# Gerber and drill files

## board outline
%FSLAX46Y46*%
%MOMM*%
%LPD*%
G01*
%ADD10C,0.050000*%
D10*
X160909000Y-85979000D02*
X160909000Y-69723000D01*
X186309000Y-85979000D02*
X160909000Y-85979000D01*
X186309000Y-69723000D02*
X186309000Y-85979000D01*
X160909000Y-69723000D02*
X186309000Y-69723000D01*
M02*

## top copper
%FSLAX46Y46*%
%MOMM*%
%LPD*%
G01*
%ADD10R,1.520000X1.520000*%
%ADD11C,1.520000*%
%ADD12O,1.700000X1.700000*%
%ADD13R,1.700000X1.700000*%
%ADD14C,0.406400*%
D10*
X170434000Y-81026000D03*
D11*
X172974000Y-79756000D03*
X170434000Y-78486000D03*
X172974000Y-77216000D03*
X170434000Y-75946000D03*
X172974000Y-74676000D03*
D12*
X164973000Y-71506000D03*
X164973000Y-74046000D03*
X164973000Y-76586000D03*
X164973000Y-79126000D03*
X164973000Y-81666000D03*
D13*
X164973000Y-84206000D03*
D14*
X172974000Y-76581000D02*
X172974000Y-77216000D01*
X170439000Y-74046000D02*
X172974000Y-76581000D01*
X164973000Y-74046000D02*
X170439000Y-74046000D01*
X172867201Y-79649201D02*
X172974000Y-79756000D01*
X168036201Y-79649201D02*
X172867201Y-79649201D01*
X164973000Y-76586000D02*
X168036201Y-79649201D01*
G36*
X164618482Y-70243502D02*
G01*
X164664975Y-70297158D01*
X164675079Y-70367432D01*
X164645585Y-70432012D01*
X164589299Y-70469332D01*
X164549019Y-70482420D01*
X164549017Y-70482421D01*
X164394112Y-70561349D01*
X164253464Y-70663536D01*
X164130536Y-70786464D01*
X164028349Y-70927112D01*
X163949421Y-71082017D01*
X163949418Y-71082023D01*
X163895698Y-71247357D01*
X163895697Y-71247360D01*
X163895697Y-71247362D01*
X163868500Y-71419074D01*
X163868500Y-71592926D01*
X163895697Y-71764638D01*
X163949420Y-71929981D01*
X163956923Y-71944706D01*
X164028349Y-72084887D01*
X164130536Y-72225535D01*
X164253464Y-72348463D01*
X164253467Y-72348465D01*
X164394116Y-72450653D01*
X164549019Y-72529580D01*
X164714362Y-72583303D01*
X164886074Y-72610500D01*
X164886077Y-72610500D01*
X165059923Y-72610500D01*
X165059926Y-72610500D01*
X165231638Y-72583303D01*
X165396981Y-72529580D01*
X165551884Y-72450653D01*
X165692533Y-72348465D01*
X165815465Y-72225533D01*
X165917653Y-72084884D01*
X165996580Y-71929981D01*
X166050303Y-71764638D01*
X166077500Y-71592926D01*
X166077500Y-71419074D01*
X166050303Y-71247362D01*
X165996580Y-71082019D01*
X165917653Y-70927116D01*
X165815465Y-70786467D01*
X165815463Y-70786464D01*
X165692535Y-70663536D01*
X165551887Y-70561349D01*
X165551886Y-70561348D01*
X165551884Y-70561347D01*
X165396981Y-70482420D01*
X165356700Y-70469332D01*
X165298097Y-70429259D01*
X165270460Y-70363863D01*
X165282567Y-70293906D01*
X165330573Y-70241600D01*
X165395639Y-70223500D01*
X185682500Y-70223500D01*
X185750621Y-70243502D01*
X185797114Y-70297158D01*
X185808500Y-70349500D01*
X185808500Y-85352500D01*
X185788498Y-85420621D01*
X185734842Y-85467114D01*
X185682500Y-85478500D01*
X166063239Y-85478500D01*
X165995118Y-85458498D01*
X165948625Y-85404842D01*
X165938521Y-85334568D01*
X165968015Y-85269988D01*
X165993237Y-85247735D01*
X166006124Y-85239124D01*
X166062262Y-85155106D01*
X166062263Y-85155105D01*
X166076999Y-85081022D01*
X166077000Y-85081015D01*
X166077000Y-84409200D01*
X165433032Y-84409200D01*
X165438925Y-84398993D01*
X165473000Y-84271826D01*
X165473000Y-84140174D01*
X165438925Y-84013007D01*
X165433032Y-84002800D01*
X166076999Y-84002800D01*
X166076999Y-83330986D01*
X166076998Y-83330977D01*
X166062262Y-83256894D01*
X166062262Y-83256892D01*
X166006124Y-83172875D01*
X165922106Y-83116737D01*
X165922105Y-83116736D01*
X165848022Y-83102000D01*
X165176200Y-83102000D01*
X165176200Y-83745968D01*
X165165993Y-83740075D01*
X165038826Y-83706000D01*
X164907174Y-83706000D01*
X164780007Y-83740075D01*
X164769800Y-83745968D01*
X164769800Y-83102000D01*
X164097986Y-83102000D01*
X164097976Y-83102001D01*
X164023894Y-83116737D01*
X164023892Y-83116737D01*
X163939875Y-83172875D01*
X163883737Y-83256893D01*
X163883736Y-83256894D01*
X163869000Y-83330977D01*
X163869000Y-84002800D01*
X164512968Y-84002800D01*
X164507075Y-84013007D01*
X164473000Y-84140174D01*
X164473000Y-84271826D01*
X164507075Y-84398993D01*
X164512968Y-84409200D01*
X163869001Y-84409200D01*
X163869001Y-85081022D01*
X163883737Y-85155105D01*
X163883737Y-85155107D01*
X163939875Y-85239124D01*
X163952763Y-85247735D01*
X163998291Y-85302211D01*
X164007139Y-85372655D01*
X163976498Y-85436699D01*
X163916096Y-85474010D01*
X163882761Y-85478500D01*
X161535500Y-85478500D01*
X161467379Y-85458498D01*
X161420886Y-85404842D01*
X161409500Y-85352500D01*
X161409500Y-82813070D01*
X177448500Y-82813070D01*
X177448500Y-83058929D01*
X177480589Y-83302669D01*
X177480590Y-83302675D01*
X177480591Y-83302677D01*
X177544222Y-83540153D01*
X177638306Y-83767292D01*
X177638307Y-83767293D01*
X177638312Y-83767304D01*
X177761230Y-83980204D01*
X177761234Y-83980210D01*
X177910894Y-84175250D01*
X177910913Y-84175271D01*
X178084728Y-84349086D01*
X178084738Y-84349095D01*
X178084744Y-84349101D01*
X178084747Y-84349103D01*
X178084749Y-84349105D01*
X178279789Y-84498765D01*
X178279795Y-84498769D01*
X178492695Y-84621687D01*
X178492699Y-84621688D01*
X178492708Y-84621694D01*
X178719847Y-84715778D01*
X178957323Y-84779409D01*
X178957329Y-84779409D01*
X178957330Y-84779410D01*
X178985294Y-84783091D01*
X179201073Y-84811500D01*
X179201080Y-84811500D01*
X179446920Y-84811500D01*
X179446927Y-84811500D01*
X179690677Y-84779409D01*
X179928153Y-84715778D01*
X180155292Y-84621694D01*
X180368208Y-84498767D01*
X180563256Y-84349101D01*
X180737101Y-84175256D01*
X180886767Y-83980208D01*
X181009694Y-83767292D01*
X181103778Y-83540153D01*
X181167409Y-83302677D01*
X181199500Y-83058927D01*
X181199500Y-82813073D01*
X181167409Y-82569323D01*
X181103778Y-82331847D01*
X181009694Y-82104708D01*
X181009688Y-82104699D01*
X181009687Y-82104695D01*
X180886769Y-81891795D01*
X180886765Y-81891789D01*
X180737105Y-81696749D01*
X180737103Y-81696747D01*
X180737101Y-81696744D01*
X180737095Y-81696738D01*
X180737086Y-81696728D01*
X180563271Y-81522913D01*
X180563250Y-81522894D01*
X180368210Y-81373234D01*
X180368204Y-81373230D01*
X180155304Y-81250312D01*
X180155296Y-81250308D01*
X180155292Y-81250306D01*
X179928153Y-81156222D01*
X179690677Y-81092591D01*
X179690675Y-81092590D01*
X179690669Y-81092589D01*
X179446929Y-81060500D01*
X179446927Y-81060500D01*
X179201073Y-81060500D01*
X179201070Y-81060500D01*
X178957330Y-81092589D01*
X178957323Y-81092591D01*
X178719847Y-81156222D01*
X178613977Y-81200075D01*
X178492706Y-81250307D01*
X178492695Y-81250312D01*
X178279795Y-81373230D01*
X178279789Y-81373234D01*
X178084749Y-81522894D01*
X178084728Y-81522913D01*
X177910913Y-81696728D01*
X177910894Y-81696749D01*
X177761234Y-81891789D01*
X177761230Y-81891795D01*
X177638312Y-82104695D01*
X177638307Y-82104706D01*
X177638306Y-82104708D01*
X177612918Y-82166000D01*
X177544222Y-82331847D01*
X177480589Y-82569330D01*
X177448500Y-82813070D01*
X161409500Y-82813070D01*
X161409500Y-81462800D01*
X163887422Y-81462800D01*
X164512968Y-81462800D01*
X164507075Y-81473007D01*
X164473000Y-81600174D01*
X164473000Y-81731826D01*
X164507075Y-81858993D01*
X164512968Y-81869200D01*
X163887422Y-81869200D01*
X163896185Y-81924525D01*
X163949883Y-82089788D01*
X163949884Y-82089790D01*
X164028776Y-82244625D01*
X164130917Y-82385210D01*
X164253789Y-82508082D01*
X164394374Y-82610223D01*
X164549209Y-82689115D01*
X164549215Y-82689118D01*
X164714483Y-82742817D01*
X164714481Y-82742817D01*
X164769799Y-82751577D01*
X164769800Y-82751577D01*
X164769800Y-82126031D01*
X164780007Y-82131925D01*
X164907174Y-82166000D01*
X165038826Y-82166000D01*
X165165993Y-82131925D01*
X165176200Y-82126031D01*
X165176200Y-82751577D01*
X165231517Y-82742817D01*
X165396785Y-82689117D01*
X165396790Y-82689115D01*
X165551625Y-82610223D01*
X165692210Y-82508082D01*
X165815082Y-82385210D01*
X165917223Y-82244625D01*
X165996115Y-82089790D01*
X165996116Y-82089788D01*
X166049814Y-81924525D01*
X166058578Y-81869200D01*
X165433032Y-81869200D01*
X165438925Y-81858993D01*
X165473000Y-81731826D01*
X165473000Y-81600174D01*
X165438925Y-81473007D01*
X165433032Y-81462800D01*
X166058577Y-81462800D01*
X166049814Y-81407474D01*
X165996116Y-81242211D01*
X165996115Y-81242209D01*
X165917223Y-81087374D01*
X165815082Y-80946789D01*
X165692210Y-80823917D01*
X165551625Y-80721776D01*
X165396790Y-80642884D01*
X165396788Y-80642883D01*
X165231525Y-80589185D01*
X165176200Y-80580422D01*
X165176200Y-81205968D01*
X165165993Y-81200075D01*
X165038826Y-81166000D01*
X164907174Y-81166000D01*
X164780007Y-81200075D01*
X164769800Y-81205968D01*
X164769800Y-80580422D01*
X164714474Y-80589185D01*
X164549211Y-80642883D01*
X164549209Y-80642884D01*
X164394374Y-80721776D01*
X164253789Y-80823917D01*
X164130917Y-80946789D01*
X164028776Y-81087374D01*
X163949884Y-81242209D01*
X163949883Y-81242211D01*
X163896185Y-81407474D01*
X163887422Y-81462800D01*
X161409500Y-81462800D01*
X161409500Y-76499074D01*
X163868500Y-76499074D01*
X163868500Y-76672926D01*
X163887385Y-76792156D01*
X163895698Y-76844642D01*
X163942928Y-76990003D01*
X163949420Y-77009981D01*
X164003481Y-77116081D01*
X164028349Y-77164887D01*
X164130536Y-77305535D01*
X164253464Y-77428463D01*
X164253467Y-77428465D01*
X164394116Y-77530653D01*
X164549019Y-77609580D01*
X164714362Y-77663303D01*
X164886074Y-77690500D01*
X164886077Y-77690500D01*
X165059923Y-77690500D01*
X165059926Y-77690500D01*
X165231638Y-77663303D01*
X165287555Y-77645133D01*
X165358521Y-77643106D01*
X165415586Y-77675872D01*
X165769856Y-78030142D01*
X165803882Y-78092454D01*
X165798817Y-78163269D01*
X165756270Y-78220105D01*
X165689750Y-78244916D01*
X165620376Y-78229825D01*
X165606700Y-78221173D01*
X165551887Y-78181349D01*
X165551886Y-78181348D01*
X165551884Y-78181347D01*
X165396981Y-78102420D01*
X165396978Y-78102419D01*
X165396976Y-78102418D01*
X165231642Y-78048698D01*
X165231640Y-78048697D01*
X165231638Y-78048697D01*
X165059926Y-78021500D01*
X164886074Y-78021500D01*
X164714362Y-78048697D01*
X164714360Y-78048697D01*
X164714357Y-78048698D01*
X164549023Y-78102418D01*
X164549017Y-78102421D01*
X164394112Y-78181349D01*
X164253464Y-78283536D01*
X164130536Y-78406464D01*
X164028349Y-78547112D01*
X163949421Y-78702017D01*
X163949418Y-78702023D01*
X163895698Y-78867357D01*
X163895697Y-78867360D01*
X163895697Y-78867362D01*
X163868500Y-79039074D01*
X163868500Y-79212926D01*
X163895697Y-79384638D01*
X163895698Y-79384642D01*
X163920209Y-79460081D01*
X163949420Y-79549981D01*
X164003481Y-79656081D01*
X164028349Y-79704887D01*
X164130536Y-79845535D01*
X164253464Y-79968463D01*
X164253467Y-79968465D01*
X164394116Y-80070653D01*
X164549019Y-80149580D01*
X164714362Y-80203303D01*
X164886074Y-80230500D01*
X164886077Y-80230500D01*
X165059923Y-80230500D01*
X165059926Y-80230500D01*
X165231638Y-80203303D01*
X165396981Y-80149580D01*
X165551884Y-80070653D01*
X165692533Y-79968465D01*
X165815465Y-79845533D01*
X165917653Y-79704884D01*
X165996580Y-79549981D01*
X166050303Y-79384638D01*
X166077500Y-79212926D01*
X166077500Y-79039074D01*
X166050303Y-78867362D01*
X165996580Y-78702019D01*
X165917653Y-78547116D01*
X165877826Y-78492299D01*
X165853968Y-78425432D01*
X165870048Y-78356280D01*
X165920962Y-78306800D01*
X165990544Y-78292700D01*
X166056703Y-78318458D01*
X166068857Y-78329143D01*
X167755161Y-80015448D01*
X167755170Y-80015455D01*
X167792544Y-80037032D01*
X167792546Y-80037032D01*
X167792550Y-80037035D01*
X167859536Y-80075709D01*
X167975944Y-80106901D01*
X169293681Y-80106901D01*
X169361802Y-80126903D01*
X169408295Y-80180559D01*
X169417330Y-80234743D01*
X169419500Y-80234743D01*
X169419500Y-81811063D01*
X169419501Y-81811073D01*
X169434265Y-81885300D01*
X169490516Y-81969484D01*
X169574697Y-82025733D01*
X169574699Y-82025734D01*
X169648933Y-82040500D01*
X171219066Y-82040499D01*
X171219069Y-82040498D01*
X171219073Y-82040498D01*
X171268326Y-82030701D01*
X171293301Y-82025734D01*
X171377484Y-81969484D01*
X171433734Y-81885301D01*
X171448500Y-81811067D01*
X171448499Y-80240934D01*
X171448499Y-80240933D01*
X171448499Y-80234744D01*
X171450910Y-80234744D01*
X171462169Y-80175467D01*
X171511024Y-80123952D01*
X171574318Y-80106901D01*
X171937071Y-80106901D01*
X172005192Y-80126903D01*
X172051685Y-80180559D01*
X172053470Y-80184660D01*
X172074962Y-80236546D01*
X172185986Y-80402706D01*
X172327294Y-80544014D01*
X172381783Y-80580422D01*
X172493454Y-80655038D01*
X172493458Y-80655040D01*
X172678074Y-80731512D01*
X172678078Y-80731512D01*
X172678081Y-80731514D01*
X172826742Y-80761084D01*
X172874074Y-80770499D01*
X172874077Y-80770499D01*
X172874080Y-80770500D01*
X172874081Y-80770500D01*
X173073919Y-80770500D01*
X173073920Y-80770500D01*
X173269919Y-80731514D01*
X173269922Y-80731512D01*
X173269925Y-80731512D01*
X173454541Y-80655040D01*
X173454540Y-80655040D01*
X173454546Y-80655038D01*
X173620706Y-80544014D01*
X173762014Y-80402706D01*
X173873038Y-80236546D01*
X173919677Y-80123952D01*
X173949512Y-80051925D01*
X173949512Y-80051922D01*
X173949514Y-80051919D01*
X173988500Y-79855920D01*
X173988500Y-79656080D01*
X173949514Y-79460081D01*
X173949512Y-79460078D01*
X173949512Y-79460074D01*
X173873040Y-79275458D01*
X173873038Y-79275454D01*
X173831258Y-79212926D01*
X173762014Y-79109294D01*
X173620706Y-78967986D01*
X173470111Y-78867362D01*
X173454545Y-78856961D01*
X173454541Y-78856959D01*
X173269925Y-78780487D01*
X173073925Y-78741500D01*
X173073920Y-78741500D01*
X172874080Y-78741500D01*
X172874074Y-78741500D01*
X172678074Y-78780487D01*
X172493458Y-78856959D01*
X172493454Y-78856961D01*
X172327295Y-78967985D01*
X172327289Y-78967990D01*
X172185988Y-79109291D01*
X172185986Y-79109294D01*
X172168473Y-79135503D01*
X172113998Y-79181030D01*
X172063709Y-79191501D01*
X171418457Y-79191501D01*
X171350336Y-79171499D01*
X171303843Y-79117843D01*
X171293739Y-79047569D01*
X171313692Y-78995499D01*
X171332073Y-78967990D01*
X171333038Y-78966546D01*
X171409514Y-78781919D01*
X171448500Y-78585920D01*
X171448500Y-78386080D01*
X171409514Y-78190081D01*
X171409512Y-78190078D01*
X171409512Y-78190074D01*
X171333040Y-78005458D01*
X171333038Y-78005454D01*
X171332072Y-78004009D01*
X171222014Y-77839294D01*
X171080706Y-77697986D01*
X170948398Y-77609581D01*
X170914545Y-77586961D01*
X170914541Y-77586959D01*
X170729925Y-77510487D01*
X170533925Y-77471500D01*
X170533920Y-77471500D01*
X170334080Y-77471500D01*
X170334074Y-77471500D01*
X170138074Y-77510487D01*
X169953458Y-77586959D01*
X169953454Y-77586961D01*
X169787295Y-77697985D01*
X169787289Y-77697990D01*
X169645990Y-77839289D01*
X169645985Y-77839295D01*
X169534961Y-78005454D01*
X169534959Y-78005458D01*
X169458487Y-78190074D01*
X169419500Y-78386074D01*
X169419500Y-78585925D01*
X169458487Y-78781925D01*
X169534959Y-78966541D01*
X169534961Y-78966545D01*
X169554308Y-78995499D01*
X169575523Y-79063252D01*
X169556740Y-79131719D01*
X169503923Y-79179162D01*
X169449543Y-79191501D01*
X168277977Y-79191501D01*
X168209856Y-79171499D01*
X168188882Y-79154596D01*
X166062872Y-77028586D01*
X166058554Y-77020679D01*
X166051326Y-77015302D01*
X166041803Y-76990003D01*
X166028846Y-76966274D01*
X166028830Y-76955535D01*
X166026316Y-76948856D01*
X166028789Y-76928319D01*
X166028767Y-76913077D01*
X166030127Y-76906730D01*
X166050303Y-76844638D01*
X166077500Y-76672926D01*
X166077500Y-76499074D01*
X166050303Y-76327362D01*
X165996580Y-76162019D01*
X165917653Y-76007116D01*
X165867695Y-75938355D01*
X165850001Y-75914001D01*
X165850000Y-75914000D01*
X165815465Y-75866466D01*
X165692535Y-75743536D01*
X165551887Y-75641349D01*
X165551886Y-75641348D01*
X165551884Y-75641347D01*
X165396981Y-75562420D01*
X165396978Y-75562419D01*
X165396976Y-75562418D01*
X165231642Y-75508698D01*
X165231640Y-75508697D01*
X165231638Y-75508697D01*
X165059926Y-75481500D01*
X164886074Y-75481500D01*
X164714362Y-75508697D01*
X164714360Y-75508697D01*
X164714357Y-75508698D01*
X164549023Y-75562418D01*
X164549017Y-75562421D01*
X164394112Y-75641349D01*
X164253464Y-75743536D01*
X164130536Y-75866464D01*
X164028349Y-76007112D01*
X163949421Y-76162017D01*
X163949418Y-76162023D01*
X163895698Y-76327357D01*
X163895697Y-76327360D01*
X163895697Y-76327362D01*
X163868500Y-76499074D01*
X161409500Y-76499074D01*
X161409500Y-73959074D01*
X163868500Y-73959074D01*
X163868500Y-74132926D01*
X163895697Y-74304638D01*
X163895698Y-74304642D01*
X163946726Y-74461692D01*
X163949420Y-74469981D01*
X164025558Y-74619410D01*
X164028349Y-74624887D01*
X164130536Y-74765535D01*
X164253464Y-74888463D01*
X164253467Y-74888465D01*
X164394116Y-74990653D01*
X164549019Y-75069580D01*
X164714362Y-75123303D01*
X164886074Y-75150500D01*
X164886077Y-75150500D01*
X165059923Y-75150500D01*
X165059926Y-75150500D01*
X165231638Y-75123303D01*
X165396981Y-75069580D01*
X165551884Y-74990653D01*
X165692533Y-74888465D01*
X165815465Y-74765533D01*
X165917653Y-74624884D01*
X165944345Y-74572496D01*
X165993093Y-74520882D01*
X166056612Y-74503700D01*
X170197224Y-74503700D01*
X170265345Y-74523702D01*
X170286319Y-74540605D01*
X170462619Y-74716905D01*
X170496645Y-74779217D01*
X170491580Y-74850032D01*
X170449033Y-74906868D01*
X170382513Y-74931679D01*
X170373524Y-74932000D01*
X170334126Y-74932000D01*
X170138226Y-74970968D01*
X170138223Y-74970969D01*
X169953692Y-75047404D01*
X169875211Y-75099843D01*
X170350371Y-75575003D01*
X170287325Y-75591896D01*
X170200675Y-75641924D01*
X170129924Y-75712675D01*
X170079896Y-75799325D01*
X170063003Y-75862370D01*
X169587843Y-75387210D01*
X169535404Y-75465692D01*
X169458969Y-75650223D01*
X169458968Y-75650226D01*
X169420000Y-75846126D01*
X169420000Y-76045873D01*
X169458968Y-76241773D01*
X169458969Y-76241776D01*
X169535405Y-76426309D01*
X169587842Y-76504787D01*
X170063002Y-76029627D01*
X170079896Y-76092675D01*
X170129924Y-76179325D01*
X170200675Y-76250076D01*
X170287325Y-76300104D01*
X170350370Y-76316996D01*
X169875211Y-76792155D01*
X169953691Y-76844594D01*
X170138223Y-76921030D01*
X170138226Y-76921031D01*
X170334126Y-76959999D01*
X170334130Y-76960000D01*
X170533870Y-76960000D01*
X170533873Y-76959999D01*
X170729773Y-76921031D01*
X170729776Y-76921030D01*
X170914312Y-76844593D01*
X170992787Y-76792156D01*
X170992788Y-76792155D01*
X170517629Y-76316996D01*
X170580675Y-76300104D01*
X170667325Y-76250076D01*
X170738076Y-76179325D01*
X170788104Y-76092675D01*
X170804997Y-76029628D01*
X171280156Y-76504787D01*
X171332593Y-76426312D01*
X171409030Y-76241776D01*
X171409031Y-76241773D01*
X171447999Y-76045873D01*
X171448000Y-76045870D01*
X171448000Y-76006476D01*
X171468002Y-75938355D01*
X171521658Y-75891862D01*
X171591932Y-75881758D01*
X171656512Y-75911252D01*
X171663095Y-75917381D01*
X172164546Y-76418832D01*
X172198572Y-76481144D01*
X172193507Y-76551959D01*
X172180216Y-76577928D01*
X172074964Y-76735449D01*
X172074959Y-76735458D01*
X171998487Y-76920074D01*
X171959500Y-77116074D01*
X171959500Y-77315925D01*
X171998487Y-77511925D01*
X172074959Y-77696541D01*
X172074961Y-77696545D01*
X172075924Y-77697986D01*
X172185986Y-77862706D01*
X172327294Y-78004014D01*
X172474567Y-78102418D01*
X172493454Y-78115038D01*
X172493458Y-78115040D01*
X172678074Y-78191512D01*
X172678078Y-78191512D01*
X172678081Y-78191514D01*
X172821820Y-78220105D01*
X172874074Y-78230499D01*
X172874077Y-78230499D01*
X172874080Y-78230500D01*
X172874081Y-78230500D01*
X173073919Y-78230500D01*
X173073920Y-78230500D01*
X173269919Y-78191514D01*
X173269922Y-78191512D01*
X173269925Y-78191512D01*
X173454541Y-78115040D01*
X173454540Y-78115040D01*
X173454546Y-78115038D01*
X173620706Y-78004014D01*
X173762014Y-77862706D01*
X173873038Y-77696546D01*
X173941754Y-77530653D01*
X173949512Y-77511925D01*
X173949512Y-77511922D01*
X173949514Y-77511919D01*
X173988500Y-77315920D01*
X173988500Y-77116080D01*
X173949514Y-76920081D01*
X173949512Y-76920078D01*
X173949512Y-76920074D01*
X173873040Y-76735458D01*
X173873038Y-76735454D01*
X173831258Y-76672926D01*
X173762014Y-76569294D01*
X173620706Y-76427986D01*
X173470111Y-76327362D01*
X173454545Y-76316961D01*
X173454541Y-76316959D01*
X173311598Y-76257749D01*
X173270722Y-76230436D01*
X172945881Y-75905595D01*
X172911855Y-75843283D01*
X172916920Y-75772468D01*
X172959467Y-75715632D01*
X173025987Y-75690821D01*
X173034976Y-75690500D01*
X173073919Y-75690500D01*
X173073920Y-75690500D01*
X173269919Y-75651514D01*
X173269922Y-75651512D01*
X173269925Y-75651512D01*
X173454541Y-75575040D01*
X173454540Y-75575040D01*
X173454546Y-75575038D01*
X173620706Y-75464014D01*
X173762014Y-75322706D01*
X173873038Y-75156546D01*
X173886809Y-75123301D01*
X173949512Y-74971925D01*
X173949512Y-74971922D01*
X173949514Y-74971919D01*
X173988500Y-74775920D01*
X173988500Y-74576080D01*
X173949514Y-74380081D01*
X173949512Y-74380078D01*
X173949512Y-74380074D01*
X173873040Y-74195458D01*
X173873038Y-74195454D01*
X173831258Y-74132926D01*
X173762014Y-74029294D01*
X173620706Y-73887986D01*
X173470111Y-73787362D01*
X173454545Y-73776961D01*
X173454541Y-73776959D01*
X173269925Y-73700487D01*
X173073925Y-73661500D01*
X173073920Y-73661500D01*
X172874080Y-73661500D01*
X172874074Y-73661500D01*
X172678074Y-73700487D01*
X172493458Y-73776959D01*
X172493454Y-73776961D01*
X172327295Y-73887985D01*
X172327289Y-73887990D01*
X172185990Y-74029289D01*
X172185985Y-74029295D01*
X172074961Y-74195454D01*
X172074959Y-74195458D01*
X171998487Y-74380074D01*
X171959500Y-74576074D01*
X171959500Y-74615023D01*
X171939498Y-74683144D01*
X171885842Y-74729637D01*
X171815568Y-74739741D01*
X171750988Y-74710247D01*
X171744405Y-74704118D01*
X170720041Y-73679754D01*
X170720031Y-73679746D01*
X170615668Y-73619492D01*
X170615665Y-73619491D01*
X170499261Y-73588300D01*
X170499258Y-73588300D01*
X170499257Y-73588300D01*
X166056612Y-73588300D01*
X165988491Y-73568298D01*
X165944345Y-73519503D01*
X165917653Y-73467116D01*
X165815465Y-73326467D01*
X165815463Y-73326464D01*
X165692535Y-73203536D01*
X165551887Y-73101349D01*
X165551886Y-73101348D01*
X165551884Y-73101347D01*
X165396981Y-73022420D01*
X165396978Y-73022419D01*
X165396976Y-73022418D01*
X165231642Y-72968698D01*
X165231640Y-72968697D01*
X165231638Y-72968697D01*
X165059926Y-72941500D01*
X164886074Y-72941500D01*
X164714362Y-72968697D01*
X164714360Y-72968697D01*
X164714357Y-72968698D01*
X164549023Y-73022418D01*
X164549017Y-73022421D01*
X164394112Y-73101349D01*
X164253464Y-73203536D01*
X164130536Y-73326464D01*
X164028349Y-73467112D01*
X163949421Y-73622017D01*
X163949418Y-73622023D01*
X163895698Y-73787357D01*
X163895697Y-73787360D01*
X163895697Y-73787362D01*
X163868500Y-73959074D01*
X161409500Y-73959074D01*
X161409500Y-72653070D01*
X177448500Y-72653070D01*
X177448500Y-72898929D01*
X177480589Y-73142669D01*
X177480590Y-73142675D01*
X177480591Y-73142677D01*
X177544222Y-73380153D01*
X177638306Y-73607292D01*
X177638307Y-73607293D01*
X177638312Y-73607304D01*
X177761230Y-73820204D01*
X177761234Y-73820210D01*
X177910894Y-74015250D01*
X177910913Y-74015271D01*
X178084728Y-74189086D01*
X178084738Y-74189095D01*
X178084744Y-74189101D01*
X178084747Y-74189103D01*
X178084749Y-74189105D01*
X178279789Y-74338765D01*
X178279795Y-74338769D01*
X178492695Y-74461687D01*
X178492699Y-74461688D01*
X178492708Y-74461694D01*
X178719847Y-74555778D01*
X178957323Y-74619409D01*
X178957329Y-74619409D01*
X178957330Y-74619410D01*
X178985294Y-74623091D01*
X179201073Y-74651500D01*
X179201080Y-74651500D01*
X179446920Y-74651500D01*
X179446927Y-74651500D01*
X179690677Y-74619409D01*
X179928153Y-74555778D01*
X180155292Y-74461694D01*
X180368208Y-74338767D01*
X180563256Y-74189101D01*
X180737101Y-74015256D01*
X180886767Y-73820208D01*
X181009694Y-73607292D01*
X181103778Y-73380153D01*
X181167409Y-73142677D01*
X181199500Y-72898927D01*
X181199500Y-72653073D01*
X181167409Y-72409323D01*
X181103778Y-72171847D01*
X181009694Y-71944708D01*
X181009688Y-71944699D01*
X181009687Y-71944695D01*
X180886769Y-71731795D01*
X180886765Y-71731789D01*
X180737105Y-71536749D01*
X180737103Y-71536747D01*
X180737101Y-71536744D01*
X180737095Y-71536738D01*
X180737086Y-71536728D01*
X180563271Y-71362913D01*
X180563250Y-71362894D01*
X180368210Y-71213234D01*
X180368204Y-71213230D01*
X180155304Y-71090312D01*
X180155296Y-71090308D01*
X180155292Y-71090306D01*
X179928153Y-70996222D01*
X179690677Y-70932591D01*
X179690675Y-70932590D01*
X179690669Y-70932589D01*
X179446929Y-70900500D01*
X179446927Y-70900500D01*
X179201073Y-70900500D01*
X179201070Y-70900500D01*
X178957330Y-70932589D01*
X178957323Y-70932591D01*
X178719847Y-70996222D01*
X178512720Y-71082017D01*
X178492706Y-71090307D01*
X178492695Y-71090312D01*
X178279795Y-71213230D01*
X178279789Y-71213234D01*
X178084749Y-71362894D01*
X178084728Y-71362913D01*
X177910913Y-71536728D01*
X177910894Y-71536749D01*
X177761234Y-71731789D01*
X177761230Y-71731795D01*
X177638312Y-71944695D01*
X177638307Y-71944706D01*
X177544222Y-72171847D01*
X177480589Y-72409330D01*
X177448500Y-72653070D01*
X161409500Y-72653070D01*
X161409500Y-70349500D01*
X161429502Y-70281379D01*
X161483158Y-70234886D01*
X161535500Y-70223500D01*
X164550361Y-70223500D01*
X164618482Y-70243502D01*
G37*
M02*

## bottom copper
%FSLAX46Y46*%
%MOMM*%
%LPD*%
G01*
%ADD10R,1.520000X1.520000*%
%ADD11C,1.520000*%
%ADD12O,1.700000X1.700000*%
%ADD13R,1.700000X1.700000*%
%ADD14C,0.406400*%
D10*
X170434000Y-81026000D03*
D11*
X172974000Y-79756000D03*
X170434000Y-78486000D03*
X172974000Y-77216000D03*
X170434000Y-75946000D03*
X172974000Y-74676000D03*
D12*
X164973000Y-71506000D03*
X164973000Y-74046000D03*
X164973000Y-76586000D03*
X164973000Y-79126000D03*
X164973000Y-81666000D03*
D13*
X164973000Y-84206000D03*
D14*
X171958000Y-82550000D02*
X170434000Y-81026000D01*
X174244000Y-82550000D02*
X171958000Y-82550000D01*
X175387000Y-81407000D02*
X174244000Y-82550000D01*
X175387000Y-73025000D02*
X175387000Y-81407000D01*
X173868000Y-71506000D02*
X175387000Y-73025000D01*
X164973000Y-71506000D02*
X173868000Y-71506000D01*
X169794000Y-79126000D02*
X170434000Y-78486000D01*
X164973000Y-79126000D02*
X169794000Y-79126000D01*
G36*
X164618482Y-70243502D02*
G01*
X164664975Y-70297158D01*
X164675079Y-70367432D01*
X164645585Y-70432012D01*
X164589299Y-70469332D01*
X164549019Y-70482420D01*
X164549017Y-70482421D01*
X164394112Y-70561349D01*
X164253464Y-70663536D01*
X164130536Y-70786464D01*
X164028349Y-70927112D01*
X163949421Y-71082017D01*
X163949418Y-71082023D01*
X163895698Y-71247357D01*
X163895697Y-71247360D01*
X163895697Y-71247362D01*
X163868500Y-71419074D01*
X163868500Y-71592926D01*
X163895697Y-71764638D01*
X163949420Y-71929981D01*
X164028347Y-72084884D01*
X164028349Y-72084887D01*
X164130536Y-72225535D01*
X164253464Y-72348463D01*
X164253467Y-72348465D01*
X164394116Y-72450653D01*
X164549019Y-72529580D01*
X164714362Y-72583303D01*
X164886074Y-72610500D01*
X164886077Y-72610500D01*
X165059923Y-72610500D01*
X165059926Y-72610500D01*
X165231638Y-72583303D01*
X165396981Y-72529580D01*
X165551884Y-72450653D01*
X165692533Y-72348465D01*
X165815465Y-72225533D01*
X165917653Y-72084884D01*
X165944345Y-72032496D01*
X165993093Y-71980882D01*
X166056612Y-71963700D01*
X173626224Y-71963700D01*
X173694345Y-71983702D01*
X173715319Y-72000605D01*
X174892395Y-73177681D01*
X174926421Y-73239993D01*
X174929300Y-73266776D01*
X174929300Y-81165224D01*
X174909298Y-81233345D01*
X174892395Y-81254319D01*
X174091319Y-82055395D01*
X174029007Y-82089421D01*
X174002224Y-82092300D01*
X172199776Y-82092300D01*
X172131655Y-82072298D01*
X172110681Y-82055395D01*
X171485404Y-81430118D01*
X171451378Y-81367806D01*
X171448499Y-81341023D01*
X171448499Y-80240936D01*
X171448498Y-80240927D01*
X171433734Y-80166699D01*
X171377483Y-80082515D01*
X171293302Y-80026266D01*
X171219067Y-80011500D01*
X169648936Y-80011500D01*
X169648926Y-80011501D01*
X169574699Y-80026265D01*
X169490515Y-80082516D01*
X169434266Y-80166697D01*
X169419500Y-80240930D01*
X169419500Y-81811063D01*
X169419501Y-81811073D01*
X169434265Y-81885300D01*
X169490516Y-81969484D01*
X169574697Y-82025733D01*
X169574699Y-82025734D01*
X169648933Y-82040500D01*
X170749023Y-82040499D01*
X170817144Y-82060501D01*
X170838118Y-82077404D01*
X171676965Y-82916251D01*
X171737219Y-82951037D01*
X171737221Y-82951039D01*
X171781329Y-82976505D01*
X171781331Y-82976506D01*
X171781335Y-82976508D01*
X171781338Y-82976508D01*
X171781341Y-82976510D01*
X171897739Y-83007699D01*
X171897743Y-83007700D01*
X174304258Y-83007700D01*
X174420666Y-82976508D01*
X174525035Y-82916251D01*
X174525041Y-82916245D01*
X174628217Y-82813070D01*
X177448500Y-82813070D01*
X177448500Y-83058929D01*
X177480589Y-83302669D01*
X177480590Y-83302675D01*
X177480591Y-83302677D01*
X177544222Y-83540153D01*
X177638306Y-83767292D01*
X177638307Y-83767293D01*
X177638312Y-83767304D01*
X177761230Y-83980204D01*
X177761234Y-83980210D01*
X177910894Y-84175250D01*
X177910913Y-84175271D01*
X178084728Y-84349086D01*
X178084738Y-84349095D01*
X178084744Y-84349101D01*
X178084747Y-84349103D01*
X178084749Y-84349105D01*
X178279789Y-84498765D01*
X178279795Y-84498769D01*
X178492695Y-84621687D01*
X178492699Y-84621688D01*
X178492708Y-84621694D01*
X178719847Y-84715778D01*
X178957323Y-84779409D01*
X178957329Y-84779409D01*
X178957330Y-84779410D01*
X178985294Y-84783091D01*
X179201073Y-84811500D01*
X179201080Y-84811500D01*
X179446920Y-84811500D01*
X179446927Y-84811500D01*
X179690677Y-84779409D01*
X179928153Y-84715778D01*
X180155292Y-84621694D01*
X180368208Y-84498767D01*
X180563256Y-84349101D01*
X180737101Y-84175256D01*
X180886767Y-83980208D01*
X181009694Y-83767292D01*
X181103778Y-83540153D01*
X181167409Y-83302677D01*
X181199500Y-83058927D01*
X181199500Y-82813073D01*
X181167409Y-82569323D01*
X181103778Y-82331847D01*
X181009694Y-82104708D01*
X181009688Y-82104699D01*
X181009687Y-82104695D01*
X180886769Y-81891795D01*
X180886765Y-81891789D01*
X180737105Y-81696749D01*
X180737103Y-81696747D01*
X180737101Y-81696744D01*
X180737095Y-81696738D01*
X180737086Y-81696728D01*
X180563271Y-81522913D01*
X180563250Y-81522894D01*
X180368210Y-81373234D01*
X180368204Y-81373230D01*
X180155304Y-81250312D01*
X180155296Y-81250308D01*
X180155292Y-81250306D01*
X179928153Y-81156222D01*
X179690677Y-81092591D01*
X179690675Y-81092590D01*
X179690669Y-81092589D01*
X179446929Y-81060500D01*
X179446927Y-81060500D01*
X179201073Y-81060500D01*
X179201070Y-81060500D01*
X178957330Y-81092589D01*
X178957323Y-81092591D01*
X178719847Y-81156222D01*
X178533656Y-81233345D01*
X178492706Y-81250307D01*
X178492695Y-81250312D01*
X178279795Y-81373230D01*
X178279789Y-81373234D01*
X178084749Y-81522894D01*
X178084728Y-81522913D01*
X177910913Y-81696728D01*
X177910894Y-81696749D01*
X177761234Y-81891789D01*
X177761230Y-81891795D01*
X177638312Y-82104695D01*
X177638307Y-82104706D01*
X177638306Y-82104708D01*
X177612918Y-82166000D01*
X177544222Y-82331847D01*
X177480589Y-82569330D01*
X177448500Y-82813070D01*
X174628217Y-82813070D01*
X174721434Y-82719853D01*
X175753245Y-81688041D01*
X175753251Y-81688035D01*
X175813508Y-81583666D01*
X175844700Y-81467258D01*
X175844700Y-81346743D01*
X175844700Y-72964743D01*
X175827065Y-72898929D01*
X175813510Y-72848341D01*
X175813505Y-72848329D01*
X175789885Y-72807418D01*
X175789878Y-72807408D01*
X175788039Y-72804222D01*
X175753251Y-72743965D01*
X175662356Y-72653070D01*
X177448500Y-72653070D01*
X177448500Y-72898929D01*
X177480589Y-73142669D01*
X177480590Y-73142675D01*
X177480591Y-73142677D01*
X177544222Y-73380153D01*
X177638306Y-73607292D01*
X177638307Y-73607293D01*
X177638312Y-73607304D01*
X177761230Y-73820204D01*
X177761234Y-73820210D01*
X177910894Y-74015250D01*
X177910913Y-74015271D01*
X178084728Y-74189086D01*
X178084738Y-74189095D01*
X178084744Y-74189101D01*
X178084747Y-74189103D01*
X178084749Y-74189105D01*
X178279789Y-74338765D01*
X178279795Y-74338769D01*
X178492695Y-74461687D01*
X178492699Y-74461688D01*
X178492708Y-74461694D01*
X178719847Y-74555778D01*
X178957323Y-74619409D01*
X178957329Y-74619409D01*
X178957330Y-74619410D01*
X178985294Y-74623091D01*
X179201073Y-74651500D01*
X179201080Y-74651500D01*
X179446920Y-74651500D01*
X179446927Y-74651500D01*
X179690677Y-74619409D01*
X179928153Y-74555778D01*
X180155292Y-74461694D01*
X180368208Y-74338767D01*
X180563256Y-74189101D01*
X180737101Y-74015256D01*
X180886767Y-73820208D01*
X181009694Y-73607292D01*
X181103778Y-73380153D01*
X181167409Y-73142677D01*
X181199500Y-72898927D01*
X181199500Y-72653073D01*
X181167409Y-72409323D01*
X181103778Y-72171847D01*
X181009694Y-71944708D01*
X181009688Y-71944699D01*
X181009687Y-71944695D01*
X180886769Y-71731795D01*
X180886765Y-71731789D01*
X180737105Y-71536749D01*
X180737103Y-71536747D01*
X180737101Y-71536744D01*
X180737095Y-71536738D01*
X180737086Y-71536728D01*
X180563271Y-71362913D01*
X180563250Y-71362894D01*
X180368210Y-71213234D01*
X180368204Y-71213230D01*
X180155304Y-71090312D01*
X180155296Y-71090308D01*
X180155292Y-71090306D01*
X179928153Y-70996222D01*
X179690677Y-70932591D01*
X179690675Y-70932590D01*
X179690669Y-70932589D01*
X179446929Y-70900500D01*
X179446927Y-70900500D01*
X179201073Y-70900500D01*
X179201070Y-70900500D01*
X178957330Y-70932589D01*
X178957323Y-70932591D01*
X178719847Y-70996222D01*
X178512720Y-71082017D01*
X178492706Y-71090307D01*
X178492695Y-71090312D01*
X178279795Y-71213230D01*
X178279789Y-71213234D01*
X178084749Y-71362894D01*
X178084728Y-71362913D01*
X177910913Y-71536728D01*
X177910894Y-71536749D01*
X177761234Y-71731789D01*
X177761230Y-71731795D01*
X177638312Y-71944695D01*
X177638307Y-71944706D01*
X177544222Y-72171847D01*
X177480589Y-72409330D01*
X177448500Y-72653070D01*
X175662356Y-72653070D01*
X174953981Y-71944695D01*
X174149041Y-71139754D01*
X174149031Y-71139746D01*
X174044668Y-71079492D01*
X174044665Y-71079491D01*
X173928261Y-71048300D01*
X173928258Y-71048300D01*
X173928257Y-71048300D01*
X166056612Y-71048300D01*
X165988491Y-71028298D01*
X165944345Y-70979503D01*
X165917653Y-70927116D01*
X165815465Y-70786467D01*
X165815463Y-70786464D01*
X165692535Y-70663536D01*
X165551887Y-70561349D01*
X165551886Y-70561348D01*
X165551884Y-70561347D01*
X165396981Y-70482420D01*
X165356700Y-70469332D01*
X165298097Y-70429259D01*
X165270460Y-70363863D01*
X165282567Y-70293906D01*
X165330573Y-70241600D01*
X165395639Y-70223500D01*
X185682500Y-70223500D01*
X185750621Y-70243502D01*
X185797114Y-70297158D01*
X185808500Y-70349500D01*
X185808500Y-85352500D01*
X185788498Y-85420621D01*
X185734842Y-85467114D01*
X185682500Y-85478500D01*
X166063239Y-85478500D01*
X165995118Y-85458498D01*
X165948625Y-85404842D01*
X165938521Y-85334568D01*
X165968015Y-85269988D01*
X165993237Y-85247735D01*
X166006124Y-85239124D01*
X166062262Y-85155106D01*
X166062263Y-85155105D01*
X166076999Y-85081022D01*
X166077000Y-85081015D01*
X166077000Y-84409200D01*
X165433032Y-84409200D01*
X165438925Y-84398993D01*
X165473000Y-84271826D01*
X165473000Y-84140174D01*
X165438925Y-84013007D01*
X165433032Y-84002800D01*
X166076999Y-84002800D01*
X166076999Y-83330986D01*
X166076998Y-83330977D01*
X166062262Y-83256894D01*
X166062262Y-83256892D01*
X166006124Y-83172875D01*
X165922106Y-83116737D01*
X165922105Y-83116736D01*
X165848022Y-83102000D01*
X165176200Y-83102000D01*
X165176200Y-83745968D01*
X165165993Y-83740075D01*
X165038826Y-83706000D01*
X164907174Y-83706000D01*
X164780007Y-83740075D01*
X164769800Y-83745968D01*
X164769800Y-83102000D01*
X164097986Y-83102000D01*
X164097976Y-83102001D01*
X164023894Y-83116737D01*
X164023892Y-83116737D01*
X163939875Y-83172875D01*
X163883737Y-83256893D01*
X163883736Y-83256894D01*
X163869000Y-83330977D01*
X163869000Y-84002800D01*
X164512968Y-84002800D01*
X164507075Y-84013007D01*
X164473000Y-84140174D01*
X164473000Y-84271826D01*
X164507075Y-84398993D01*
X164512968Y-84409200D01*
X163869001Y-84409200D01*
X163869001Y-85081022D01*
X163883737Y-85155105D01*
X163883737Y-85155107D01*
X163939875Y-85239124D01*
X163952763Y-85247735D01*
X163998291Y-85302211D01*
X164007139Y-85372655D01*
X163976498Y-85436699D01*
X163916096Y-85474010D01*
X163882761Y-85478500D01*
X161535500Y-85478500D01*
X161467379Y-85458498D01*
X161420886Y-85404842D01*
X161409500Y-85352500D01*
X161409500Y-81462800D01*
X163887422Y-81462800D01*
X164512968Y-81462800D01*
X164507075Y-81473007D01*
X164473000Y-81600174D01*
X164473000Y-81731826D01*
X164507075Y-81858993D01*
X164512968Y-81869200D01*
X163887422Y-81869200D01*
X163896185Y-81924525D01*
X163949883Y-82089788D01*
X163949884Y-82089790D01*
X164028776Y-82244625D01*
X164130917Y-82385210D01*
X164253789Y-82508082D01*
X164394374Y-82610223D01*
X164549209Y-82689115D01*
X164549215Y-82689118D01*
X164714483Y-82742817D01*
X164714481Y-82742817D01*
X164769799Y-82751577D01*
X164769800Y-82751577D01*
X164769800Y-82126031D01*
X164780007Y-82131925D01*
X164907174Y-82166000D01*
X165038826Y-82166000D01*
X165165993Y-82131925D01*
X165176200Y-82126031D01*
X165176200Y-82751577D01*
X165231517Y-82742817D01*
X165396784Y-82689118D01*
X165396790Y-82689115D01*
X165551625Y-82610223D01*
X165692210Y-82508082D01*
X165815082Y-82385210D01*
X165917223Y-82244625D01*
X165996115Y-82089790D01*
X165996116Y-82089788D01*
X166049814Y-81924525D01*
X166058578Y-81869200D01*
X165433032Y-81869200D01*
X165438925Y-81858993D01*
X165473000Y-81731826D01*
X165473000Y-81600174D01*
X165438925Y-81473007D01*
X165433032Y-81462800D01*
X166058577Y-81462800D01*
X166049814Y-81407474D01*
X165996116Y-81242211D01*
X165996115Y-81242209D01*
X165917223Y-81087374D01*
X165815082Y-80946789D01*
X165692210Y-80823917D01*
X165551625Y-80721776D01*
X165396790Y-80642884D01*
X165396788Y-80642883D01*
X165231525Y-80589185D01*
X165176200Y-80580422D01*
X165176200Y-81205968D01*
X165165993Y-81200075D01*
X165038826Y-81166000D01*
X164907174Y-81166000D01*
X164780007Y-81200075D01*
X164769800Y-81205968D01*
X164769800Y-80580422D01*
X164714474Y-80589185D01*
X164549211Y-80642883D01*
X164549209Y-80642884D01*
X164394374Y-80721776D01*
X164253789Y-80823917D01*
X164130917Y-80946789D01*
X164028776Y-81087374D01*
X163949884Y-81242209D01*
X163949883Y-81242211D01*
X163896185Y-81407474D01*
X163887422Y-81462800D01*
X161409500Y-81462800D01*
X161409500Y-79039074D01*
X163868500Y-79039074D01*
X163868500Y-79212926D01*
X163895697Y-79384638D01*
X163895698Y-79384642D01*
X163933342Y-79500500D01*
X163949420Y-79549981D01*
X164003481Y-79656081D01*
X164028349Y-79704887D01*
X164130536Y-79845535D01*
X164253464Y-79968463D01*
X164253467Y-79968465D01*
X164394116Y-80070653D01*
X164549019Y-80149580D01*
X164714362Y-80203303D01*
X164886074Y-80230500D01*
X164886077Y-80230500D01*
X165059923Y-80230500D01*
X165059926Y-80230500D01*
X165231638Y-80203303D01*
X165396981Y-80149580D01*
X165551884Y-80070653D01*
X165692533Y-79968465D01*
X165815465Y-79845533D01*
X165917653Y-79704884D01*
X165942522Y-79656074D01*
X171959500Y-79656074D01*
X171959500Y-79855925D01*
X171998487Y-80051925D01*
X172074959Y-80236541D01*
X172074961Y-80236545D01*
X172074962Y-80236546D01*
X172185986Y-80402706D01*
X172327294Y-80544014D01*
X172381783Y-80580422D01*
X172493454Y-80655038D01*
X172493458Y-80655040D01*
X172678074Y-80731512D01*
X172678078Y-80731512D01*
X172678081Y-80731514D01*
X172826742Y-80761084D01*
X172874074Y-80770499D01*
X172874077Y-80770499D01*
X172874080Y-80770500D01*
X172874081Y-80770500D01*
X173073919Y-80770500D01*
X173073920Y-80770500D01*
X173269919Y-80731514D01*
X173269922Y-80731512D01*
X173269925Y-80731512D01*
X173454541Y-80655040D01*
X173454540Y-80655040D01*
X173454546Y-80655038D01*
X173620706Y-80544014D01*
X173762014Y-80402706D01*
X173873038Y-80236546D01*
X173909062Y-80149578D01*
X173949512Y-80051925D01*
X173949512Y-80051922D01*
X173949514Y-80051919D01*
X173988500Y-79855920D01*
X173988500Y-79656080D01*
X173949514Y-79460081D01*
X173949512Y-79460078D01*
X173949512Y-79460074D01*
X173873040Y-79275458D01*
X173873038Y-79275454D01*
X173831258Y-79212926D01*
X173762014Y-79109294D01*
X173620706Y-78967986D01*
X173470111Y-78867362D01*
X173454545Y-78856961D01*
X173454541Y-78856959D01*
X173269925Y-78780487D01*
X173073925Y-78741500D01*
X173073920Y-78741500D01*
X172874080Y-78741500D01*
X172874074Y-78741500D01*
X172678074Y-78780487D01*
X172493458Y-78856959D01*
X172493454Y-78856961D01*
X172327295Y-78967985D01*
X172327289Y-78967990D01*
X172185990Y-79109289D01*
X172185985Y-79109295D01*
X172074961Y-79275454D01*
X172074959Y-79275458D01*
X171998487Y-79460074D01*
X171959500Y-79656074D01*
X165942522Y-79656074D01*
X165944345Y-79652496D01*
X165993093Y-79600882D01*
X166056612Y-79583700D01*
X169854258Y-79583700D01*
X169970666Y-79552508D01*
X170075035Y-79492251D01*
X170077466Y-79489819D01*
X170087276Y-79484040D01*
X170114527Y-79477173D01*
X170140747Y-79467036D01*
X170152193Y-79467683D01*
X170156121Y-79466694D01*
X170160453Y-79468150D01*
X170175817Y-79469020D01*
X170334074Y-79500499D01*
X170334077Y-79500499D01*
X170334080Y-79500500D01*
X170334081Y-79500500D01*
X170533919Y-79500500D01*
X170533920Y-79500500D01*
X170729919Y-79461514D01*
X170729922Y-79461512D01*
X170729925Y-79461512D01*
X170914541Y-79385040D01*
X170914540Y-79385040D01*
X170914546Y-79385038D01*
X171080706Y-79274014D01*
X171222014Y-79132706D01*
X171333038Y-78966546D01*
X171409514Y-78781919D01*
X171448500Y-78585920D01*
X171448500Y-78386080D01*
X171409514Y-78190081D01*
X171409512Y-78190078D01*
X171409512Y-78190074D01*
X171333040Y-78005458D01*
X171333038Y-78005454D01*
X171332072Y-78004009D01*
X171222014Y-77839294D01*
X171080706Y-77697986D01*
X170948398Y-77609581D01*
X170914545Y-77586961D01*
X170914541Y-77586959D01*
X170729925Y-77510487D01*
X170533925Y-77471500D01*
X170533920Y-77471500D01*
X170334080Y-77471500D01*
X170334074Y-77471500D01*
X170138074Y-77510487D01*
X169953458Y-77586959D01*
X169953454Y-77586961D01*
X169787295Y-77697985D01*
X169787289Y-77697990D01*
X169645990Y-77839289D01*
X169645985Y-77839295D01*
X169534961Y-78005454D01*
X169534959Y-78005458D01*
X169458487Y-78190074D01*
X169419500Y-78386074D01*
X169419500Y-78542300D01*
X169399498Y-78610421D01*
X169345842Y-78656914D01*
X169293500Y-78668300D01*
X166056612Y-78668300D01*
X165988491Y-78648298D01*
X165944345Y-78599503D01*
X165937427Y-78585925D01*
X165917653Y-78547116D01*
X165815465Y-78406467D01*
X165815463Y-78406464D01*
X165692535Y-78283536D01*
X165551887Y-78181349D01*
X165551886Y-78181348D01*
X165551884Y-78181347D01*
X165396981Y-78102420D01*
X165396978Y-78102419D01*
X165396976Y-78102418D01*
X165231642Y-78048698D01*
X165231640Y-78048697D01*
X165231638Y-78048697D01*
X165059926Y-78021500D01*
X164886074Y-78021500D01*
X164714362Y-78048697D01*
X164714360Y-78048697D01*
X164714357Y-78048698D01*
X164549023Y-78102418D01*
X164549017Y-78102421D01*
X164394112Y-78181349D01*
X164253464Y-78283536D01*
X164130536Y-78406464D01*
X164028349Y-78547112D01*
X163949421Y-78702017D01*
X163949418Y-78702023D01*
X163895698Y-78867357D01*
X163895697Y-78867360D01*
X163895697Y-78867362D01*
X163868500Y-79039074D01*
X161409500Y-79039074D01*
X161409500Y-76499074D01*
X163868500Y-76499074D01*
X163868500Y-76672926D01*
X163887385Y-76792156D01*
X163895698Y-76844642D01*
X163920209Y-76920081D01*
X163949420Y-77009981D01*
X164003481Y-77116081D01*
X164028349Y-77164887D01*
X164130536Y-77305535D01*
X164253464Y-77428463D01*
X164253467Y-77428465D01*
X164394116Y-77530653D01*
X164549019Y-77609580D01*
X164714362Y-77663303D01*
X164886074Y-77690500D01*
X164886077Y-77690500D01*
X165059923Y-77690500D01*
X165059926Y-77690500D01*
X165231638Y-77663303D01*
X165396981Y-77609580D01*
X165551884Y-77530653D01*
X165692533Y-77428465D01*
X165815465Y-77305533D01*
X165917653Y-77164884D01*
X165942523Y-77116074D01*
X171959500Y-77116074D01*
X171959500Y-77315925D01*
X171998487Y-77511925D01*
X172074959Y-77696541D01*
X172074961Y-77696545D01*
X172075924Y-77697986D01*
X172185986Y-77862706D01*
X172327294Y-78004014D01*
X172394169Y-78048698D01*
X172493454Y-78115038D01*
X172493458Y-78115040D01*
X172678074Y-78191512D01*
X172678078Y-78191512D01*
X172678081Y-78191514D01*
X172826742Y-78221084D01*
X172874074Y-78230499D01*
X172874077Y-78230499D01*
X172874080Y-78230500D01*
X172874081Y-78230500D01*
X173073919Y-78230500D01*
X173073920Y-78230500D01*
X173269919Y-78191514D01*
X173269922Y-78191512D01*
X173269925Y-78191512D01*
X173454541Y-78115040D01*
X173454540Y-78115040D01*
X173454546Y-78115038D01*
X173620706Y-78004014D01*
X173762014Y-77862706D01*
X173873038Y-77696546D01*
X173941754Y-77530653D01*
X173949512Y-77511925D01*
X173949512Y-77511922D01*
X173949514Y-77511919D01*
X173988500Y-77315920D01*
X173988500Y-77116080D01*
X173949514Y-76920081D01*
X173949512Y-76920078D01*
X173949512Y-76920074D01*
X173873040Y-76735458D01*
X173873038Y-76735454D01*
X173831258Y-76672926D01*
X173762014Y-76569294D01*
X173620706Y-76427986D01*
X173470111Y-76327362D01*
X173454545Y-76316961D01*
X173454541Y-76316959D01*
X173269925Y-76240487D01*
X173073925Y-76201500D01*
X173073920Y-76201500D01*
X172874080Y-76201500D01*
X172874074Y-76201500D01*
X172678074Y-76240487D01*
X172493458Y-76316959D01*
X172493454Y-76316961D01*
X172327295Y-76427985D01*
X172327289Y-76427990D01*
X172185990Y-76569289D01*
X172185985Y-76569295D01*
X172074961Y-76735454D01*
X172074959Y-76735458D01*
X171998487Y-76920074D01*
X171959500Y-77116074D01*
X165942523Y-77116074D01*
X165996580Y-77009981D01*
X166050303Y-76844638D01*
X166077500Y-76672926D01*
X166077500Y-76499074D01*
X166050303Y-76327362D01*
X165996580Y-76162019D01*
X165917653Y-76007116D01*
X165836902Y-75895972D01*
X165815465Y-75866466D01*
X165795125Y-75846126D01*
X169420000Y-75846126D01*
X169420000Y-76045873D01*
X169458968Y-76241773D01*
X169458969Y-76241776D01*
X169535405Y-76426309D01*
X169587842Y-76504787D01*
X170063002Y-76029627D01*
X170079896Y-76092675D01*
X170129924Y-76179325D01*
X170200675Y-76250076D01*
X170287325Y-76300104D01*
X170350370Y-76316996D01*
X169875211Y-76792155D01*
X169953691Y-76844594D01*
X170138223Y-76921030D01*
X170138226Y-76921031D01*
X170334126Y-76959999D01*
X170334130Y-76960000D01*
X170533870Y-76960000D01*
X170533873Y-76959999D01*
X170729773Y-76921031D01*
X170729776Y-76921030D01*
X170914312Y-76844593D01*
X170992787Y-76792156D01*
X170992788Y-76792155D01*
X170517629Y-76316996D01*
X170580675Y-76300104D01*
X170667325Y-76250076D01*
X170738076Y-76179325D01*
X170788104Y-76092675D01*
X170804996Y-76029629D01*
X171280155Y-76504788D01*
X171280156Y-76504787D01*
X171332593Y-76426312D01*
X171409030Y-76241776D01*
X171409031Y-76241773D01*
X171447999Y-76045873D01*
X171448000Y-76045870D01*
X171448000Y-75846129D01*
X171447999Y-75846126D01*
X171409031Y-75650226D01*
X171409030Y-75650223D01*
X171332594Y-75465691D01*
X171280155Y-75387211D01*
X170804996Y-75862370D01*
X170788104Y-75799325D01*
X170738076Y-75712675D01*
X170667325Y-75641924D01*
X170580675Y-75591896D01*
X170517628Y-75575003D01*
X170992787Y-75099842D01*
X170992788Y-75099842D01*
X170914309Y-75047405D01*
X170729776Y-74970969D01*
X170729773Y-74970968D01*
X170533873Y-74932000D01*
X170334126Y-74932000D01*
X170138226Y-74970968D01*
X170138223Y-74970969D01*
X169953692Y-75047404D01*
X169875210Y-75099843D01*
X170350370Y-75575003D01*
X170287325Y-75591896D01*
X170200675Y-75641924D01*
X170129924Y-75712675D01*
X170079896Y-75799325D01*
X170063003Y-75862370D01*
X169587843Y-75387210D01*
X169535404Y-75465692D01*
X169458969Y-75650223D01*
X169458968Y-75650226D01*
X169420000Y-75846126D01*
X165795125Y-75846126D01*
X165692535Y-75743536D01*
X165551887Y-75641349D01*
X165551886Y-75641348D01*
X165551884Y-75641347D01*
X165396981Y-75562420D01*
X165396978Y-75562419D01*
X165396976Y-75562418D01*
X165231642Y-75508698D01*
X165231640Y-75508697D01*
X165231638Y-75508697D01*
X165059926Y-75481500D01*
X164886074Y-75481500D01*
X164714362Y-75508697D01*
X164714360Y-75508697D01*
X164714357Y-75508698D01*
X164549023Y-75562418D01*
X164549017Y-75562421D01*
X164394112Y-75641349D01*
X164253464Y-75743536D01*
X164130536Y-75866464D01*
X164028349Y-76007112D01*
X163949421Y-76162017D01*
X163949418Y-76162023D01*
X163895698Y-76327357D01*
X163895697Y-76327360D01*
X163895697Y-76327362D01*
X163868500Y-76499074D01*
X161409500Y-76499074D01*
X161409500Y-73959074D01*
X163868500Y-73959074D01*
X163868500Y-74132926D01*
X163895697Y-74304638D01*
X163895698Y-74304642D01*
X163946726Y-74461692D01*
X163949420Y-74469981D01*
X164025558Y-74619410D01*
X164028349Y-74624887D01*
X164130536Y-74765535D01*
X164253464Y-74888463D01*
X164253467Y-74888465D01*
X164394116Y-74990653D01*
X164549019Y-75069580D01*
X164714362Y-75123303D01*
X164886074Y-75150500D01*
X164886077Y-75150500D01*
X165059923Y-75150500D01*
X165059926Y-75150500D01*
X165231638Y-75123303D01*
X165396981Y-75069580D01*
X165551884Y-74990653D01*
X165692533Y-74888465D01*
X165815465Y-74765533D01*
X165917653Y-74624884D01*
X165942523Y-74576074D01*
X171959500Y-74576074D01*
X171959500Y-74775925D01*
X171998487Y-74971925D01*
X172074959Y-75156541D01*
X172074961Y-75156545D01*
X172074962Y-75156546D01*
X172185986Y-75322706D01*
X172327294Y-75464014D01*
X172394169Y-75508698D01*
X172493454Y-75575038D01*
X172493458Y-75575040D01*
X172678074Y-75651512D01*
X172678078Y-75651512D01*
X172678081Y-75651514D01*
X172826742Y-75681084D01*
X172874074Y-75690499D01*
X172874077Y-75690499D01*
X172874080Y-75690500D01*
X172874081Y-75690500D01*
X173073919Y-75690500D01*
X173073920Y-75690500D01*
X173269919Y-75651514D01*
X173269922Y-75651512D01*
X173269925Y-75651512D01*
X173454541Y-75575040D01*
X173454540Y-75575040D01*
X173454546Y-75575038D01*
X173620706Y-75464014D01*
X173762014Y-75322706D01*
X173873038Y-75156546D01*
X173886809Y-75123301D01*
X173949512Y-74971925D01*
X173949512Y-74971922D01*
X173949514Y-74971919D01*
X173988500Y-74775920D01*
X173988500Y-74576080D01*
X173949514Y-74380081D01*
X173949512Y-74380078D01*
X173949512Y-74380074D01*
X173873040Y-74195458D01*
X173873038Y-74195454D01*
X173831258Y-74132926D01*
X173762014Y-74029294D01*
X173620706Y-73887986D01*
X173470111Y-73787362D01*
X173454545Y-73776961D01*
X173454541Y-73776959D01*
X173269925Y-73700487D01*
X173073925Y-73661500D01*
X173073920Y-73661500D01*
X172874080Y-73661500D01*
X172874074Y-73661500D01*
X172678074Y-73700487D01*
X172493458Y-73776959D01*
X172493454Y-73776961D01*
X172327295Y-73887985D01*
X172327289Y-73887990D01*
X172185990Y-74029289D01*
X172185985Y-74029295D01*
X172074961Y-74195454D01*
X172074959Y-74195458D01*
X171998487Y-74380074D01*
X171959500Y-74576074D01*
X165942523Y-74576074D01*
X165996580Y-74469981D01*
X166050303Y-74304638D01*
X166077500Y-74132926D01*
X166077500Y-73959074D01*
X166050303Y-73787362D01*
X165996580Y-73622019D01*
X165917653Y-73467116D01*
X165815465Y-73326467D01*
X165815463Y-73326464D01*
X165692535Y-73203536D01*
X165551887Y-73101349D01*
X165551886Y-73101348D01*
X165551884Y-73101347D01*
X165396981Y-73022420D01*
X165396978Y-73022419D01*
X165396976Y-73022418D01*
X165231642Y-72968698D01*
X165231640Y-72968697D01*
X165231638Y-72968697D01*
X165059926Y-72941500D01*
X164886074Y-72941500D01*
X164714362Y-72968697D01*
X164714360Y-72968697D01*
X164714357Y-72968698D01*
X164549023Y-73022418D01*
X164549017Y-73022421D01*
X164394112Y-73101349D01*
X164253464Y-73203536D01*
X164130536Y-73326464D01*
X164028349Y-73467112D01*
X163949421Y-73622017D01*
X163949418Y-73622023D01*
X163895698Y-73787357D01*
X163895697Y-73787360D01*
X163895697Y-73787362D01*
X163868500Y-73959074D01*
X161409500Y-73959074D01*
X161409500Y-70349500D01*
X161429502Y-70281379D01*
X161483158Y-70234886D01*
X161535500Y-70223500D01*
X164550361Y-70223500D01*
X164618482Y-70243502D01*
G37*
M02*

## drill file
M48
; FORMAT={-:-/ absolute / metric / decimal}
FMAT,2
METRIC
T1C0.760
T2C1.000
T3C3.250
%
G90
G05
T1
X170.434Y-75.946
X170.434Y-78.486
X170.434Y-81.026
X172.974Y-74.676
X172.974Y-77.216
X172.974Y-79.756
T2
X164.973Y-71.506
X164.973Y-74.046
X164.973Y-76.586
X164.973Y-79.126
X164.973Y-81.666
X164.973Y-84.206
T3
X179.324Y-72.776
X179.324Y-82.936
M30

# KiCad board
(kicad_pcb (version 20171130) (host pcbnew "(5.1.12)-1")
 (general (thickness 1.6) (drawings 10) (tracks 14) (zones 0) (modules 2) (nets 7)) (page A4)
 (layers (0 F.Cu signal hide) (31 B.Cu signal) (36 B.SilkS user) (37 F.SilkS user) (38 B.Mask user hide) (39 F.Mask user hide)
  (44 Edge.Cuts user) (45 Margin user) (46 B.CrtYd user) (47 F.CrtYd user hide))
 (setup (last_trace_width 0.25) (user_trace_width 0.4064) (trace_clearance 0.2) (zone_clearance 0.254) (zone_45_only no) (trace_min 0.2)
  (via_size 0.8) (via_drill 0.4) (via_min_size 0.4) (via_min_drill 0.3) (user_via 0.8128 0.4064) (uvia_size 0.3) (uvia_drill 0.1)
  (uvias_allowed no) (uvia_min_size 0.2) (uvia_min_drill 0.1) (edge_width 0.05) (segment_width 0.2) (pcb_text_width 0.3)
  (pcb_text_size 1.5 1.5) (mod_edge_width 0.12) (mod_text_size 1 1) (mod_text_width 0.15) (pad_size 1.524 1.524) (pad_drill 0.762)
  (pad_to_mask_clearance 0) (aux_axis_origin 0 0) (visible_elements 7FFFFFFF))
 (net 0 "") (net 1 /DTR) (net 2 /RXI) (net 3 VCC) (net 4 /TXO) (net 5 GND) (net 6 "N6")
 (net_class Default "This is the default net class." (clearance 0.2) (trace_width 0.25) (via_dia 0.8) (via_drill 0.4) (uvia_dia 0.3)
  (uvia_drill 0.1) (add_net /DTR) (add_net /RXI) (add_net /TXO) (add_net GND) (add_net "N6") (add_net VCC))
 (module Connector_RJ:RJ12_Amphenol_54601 (layer F.Cu) (at 170.434 81.026 90)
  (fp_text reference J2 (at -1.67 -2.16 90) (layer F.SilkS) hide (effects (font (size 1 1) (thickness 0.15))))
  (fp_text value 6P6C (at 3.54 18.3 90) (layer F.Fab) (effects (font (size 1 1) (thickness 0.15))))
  (pad 1 thru_hole rect (at 0 0 90) (size 1.52 1.52) (drill 0.76) (layers *.Cu *.Mask) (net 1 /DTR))
  (pad "" np_thru_hole circle (at -1.91 8.89 90) (size 3.25 3.25) (drill 3.25) (layers *.Cu *.Mask))
  (pad 2 thru_hole circle (at 1.27 2.54 90) (size 1.52 1.52) (drill 0.76) (layers *.Cu *.Mask) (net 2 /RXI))
  (pad 3 thru_hole circle (at 2.54 0 90) (size 1.52 1.52) (drill 0.76) (layers *.Cu *.Mask) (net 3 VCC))
  (pad 4 thru_hole circle (at 3.81 2.54 90) (size 1.52 1.52) (drill 0.76) (layers *.Cu *.Mask) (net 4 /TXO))
  (pad 5 thru_hole circle (at 5.08 0 90) (size 1.52 1.52) (drill 0.76) (layers *.Cu *.Mask) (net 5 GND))
  (pad 6 thru_hole circle (at 6.35 2.54 90) (size 1.52 1.52) (drill 0.76) (layers *.Cu *.Mask) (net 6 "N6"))
  (pad "" np_thru_hole circle (at 8.25 8.89 90) (size 3.25 3.25) (drill 3.25) (layers *.Cu *.Mask)))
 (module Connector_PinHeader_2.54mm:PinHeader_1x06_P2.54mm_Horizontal (layer F.Cu) (at 164.973 84.206 180)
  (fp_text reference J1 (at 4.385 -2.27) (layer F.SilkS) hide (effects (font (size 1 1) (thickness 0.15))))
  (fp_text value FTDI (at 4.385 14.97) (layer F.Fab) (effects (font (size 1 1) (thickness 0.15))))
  (pad 6 thru_hole oval (at 0 12.7 180) (size 1.7 1.7) (drill 1) (layers *.Cu *.Mask) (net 1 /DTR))
  (pad 5 thru_hole oval (at 0 10.16 180) (size 1.7 1.7) (drill 1) (layers *.Cu *.Mask) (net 4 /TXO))
  (pad 4 thru_hole oval (at 0 7.62 180) (size 1.7 1.7) (drill 1) (layers *.Cu *.Mask) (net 2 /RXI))
  (pad 3 thru_hole oval (at 0 5.08 180) (size 1.7 1.7) (drill 1) (layers *.Cu *.Mask) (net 3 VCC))
  (pad 2 thru_hole oval (at 0 2.54 180) (size 1.7 1.7) (drill 1) (layers *.Cu *.Mask) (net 5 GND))
  (pad 1 thru_hole rect (at 0 0 180) (size 1.7 1.7) (drill 1) (layers *.Cu *.Mask) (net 5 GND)))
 (gr_line (start 160.909 85.979) (end 160.909 69.723) (layer Edge.Cuts) (width 0.05))
 (gr_line (start 186.309 85.979) (end 160.909 85.979) (layer Edge.Cuts) (width 0.05))
 (gr_line (start 186.309 69.723) (end 186.309 85.979) (layer Edge.Cuts) (width 0.05))
 (gr_line (start 160.909 69.723) (end 186.309 69.723) (layer Edge.Cuts) (width 0.05))
 (segment (start 171.958 82.55) (end 170.434 81.026) (width 0.4064) (layer B.Cu) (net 1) (status 20))
 (segment (start 174.244 82.55) (end 171.958 82.55) (width 0.4064) (layer B.Cu) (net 1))
 (segment (start 175.387 81.407) (end 174.244 82.55) (width 0.4064) (layer B.Cu) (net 1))
 (segment (start 175.387 73.025) (end 175.387 81.407) (width 0.4064) (layer B.Cu) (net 1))
 (segment (start 173.868 71.506) (end 175.387 73.025) (width 0.4064) (layer B.Cu) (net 1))
 (segment (start 164.973 71.506) (end 173.868 71.506) (width 0.4064) (layer B.Cu) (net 1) (status 10))
 (segment (start 172.974 76.581) (end 172.974 77.216) (width 0.4064) (layer F.Cu) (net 4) (status 30))
 (segment (start 170.439 74.046) (end 172.974 76.581) (width 0.4064) (layer F.Cu) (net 4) (status 20))
 (segment (start 164.973 74.046) (end 170.439 74.046) (width 0.4064) (layer F.Cu) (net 4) (status 10))
 (segment (start 172.867201 79.649201) (end 172.974 79.756) (width 0.4064) (layer F.Cu) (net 2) (status 30))
 (segment (start 168.036201 79.649201) (end 172.867201 79.649201) (width 0.4064) (layer F.Cu) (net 2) (status 20))
 (segment (start 164.973 76.586) (end 168.036201 79.649201) (width 0.4064) (layer F.Cu) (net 2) (status 10))
 (segment (start 169.794 79.126) (end 170.434 78.486) (width 0.4064) (layer B.Cu) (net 3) (status 20))
 (segment (start 164.973 79.126) (end 169.794 79.126) (width 0.4064) (layer B.Cu) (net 3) (status 10))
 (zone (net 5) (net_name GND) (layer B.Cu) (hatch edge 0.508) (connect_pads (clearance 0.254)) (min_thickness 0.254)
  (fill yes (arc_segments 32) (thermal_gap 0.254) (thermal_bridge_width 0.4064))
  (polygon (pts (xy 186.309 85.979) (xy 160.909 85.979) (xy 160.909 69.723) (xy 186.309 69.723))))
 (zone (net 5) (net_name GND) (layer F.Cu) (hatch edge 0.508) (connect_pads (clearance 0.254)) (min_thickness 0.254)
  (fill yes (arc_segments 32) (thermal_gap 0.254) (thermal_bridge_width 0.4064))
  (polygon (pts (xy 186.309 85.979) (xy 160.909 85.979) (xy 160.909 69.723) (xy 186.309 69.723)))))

